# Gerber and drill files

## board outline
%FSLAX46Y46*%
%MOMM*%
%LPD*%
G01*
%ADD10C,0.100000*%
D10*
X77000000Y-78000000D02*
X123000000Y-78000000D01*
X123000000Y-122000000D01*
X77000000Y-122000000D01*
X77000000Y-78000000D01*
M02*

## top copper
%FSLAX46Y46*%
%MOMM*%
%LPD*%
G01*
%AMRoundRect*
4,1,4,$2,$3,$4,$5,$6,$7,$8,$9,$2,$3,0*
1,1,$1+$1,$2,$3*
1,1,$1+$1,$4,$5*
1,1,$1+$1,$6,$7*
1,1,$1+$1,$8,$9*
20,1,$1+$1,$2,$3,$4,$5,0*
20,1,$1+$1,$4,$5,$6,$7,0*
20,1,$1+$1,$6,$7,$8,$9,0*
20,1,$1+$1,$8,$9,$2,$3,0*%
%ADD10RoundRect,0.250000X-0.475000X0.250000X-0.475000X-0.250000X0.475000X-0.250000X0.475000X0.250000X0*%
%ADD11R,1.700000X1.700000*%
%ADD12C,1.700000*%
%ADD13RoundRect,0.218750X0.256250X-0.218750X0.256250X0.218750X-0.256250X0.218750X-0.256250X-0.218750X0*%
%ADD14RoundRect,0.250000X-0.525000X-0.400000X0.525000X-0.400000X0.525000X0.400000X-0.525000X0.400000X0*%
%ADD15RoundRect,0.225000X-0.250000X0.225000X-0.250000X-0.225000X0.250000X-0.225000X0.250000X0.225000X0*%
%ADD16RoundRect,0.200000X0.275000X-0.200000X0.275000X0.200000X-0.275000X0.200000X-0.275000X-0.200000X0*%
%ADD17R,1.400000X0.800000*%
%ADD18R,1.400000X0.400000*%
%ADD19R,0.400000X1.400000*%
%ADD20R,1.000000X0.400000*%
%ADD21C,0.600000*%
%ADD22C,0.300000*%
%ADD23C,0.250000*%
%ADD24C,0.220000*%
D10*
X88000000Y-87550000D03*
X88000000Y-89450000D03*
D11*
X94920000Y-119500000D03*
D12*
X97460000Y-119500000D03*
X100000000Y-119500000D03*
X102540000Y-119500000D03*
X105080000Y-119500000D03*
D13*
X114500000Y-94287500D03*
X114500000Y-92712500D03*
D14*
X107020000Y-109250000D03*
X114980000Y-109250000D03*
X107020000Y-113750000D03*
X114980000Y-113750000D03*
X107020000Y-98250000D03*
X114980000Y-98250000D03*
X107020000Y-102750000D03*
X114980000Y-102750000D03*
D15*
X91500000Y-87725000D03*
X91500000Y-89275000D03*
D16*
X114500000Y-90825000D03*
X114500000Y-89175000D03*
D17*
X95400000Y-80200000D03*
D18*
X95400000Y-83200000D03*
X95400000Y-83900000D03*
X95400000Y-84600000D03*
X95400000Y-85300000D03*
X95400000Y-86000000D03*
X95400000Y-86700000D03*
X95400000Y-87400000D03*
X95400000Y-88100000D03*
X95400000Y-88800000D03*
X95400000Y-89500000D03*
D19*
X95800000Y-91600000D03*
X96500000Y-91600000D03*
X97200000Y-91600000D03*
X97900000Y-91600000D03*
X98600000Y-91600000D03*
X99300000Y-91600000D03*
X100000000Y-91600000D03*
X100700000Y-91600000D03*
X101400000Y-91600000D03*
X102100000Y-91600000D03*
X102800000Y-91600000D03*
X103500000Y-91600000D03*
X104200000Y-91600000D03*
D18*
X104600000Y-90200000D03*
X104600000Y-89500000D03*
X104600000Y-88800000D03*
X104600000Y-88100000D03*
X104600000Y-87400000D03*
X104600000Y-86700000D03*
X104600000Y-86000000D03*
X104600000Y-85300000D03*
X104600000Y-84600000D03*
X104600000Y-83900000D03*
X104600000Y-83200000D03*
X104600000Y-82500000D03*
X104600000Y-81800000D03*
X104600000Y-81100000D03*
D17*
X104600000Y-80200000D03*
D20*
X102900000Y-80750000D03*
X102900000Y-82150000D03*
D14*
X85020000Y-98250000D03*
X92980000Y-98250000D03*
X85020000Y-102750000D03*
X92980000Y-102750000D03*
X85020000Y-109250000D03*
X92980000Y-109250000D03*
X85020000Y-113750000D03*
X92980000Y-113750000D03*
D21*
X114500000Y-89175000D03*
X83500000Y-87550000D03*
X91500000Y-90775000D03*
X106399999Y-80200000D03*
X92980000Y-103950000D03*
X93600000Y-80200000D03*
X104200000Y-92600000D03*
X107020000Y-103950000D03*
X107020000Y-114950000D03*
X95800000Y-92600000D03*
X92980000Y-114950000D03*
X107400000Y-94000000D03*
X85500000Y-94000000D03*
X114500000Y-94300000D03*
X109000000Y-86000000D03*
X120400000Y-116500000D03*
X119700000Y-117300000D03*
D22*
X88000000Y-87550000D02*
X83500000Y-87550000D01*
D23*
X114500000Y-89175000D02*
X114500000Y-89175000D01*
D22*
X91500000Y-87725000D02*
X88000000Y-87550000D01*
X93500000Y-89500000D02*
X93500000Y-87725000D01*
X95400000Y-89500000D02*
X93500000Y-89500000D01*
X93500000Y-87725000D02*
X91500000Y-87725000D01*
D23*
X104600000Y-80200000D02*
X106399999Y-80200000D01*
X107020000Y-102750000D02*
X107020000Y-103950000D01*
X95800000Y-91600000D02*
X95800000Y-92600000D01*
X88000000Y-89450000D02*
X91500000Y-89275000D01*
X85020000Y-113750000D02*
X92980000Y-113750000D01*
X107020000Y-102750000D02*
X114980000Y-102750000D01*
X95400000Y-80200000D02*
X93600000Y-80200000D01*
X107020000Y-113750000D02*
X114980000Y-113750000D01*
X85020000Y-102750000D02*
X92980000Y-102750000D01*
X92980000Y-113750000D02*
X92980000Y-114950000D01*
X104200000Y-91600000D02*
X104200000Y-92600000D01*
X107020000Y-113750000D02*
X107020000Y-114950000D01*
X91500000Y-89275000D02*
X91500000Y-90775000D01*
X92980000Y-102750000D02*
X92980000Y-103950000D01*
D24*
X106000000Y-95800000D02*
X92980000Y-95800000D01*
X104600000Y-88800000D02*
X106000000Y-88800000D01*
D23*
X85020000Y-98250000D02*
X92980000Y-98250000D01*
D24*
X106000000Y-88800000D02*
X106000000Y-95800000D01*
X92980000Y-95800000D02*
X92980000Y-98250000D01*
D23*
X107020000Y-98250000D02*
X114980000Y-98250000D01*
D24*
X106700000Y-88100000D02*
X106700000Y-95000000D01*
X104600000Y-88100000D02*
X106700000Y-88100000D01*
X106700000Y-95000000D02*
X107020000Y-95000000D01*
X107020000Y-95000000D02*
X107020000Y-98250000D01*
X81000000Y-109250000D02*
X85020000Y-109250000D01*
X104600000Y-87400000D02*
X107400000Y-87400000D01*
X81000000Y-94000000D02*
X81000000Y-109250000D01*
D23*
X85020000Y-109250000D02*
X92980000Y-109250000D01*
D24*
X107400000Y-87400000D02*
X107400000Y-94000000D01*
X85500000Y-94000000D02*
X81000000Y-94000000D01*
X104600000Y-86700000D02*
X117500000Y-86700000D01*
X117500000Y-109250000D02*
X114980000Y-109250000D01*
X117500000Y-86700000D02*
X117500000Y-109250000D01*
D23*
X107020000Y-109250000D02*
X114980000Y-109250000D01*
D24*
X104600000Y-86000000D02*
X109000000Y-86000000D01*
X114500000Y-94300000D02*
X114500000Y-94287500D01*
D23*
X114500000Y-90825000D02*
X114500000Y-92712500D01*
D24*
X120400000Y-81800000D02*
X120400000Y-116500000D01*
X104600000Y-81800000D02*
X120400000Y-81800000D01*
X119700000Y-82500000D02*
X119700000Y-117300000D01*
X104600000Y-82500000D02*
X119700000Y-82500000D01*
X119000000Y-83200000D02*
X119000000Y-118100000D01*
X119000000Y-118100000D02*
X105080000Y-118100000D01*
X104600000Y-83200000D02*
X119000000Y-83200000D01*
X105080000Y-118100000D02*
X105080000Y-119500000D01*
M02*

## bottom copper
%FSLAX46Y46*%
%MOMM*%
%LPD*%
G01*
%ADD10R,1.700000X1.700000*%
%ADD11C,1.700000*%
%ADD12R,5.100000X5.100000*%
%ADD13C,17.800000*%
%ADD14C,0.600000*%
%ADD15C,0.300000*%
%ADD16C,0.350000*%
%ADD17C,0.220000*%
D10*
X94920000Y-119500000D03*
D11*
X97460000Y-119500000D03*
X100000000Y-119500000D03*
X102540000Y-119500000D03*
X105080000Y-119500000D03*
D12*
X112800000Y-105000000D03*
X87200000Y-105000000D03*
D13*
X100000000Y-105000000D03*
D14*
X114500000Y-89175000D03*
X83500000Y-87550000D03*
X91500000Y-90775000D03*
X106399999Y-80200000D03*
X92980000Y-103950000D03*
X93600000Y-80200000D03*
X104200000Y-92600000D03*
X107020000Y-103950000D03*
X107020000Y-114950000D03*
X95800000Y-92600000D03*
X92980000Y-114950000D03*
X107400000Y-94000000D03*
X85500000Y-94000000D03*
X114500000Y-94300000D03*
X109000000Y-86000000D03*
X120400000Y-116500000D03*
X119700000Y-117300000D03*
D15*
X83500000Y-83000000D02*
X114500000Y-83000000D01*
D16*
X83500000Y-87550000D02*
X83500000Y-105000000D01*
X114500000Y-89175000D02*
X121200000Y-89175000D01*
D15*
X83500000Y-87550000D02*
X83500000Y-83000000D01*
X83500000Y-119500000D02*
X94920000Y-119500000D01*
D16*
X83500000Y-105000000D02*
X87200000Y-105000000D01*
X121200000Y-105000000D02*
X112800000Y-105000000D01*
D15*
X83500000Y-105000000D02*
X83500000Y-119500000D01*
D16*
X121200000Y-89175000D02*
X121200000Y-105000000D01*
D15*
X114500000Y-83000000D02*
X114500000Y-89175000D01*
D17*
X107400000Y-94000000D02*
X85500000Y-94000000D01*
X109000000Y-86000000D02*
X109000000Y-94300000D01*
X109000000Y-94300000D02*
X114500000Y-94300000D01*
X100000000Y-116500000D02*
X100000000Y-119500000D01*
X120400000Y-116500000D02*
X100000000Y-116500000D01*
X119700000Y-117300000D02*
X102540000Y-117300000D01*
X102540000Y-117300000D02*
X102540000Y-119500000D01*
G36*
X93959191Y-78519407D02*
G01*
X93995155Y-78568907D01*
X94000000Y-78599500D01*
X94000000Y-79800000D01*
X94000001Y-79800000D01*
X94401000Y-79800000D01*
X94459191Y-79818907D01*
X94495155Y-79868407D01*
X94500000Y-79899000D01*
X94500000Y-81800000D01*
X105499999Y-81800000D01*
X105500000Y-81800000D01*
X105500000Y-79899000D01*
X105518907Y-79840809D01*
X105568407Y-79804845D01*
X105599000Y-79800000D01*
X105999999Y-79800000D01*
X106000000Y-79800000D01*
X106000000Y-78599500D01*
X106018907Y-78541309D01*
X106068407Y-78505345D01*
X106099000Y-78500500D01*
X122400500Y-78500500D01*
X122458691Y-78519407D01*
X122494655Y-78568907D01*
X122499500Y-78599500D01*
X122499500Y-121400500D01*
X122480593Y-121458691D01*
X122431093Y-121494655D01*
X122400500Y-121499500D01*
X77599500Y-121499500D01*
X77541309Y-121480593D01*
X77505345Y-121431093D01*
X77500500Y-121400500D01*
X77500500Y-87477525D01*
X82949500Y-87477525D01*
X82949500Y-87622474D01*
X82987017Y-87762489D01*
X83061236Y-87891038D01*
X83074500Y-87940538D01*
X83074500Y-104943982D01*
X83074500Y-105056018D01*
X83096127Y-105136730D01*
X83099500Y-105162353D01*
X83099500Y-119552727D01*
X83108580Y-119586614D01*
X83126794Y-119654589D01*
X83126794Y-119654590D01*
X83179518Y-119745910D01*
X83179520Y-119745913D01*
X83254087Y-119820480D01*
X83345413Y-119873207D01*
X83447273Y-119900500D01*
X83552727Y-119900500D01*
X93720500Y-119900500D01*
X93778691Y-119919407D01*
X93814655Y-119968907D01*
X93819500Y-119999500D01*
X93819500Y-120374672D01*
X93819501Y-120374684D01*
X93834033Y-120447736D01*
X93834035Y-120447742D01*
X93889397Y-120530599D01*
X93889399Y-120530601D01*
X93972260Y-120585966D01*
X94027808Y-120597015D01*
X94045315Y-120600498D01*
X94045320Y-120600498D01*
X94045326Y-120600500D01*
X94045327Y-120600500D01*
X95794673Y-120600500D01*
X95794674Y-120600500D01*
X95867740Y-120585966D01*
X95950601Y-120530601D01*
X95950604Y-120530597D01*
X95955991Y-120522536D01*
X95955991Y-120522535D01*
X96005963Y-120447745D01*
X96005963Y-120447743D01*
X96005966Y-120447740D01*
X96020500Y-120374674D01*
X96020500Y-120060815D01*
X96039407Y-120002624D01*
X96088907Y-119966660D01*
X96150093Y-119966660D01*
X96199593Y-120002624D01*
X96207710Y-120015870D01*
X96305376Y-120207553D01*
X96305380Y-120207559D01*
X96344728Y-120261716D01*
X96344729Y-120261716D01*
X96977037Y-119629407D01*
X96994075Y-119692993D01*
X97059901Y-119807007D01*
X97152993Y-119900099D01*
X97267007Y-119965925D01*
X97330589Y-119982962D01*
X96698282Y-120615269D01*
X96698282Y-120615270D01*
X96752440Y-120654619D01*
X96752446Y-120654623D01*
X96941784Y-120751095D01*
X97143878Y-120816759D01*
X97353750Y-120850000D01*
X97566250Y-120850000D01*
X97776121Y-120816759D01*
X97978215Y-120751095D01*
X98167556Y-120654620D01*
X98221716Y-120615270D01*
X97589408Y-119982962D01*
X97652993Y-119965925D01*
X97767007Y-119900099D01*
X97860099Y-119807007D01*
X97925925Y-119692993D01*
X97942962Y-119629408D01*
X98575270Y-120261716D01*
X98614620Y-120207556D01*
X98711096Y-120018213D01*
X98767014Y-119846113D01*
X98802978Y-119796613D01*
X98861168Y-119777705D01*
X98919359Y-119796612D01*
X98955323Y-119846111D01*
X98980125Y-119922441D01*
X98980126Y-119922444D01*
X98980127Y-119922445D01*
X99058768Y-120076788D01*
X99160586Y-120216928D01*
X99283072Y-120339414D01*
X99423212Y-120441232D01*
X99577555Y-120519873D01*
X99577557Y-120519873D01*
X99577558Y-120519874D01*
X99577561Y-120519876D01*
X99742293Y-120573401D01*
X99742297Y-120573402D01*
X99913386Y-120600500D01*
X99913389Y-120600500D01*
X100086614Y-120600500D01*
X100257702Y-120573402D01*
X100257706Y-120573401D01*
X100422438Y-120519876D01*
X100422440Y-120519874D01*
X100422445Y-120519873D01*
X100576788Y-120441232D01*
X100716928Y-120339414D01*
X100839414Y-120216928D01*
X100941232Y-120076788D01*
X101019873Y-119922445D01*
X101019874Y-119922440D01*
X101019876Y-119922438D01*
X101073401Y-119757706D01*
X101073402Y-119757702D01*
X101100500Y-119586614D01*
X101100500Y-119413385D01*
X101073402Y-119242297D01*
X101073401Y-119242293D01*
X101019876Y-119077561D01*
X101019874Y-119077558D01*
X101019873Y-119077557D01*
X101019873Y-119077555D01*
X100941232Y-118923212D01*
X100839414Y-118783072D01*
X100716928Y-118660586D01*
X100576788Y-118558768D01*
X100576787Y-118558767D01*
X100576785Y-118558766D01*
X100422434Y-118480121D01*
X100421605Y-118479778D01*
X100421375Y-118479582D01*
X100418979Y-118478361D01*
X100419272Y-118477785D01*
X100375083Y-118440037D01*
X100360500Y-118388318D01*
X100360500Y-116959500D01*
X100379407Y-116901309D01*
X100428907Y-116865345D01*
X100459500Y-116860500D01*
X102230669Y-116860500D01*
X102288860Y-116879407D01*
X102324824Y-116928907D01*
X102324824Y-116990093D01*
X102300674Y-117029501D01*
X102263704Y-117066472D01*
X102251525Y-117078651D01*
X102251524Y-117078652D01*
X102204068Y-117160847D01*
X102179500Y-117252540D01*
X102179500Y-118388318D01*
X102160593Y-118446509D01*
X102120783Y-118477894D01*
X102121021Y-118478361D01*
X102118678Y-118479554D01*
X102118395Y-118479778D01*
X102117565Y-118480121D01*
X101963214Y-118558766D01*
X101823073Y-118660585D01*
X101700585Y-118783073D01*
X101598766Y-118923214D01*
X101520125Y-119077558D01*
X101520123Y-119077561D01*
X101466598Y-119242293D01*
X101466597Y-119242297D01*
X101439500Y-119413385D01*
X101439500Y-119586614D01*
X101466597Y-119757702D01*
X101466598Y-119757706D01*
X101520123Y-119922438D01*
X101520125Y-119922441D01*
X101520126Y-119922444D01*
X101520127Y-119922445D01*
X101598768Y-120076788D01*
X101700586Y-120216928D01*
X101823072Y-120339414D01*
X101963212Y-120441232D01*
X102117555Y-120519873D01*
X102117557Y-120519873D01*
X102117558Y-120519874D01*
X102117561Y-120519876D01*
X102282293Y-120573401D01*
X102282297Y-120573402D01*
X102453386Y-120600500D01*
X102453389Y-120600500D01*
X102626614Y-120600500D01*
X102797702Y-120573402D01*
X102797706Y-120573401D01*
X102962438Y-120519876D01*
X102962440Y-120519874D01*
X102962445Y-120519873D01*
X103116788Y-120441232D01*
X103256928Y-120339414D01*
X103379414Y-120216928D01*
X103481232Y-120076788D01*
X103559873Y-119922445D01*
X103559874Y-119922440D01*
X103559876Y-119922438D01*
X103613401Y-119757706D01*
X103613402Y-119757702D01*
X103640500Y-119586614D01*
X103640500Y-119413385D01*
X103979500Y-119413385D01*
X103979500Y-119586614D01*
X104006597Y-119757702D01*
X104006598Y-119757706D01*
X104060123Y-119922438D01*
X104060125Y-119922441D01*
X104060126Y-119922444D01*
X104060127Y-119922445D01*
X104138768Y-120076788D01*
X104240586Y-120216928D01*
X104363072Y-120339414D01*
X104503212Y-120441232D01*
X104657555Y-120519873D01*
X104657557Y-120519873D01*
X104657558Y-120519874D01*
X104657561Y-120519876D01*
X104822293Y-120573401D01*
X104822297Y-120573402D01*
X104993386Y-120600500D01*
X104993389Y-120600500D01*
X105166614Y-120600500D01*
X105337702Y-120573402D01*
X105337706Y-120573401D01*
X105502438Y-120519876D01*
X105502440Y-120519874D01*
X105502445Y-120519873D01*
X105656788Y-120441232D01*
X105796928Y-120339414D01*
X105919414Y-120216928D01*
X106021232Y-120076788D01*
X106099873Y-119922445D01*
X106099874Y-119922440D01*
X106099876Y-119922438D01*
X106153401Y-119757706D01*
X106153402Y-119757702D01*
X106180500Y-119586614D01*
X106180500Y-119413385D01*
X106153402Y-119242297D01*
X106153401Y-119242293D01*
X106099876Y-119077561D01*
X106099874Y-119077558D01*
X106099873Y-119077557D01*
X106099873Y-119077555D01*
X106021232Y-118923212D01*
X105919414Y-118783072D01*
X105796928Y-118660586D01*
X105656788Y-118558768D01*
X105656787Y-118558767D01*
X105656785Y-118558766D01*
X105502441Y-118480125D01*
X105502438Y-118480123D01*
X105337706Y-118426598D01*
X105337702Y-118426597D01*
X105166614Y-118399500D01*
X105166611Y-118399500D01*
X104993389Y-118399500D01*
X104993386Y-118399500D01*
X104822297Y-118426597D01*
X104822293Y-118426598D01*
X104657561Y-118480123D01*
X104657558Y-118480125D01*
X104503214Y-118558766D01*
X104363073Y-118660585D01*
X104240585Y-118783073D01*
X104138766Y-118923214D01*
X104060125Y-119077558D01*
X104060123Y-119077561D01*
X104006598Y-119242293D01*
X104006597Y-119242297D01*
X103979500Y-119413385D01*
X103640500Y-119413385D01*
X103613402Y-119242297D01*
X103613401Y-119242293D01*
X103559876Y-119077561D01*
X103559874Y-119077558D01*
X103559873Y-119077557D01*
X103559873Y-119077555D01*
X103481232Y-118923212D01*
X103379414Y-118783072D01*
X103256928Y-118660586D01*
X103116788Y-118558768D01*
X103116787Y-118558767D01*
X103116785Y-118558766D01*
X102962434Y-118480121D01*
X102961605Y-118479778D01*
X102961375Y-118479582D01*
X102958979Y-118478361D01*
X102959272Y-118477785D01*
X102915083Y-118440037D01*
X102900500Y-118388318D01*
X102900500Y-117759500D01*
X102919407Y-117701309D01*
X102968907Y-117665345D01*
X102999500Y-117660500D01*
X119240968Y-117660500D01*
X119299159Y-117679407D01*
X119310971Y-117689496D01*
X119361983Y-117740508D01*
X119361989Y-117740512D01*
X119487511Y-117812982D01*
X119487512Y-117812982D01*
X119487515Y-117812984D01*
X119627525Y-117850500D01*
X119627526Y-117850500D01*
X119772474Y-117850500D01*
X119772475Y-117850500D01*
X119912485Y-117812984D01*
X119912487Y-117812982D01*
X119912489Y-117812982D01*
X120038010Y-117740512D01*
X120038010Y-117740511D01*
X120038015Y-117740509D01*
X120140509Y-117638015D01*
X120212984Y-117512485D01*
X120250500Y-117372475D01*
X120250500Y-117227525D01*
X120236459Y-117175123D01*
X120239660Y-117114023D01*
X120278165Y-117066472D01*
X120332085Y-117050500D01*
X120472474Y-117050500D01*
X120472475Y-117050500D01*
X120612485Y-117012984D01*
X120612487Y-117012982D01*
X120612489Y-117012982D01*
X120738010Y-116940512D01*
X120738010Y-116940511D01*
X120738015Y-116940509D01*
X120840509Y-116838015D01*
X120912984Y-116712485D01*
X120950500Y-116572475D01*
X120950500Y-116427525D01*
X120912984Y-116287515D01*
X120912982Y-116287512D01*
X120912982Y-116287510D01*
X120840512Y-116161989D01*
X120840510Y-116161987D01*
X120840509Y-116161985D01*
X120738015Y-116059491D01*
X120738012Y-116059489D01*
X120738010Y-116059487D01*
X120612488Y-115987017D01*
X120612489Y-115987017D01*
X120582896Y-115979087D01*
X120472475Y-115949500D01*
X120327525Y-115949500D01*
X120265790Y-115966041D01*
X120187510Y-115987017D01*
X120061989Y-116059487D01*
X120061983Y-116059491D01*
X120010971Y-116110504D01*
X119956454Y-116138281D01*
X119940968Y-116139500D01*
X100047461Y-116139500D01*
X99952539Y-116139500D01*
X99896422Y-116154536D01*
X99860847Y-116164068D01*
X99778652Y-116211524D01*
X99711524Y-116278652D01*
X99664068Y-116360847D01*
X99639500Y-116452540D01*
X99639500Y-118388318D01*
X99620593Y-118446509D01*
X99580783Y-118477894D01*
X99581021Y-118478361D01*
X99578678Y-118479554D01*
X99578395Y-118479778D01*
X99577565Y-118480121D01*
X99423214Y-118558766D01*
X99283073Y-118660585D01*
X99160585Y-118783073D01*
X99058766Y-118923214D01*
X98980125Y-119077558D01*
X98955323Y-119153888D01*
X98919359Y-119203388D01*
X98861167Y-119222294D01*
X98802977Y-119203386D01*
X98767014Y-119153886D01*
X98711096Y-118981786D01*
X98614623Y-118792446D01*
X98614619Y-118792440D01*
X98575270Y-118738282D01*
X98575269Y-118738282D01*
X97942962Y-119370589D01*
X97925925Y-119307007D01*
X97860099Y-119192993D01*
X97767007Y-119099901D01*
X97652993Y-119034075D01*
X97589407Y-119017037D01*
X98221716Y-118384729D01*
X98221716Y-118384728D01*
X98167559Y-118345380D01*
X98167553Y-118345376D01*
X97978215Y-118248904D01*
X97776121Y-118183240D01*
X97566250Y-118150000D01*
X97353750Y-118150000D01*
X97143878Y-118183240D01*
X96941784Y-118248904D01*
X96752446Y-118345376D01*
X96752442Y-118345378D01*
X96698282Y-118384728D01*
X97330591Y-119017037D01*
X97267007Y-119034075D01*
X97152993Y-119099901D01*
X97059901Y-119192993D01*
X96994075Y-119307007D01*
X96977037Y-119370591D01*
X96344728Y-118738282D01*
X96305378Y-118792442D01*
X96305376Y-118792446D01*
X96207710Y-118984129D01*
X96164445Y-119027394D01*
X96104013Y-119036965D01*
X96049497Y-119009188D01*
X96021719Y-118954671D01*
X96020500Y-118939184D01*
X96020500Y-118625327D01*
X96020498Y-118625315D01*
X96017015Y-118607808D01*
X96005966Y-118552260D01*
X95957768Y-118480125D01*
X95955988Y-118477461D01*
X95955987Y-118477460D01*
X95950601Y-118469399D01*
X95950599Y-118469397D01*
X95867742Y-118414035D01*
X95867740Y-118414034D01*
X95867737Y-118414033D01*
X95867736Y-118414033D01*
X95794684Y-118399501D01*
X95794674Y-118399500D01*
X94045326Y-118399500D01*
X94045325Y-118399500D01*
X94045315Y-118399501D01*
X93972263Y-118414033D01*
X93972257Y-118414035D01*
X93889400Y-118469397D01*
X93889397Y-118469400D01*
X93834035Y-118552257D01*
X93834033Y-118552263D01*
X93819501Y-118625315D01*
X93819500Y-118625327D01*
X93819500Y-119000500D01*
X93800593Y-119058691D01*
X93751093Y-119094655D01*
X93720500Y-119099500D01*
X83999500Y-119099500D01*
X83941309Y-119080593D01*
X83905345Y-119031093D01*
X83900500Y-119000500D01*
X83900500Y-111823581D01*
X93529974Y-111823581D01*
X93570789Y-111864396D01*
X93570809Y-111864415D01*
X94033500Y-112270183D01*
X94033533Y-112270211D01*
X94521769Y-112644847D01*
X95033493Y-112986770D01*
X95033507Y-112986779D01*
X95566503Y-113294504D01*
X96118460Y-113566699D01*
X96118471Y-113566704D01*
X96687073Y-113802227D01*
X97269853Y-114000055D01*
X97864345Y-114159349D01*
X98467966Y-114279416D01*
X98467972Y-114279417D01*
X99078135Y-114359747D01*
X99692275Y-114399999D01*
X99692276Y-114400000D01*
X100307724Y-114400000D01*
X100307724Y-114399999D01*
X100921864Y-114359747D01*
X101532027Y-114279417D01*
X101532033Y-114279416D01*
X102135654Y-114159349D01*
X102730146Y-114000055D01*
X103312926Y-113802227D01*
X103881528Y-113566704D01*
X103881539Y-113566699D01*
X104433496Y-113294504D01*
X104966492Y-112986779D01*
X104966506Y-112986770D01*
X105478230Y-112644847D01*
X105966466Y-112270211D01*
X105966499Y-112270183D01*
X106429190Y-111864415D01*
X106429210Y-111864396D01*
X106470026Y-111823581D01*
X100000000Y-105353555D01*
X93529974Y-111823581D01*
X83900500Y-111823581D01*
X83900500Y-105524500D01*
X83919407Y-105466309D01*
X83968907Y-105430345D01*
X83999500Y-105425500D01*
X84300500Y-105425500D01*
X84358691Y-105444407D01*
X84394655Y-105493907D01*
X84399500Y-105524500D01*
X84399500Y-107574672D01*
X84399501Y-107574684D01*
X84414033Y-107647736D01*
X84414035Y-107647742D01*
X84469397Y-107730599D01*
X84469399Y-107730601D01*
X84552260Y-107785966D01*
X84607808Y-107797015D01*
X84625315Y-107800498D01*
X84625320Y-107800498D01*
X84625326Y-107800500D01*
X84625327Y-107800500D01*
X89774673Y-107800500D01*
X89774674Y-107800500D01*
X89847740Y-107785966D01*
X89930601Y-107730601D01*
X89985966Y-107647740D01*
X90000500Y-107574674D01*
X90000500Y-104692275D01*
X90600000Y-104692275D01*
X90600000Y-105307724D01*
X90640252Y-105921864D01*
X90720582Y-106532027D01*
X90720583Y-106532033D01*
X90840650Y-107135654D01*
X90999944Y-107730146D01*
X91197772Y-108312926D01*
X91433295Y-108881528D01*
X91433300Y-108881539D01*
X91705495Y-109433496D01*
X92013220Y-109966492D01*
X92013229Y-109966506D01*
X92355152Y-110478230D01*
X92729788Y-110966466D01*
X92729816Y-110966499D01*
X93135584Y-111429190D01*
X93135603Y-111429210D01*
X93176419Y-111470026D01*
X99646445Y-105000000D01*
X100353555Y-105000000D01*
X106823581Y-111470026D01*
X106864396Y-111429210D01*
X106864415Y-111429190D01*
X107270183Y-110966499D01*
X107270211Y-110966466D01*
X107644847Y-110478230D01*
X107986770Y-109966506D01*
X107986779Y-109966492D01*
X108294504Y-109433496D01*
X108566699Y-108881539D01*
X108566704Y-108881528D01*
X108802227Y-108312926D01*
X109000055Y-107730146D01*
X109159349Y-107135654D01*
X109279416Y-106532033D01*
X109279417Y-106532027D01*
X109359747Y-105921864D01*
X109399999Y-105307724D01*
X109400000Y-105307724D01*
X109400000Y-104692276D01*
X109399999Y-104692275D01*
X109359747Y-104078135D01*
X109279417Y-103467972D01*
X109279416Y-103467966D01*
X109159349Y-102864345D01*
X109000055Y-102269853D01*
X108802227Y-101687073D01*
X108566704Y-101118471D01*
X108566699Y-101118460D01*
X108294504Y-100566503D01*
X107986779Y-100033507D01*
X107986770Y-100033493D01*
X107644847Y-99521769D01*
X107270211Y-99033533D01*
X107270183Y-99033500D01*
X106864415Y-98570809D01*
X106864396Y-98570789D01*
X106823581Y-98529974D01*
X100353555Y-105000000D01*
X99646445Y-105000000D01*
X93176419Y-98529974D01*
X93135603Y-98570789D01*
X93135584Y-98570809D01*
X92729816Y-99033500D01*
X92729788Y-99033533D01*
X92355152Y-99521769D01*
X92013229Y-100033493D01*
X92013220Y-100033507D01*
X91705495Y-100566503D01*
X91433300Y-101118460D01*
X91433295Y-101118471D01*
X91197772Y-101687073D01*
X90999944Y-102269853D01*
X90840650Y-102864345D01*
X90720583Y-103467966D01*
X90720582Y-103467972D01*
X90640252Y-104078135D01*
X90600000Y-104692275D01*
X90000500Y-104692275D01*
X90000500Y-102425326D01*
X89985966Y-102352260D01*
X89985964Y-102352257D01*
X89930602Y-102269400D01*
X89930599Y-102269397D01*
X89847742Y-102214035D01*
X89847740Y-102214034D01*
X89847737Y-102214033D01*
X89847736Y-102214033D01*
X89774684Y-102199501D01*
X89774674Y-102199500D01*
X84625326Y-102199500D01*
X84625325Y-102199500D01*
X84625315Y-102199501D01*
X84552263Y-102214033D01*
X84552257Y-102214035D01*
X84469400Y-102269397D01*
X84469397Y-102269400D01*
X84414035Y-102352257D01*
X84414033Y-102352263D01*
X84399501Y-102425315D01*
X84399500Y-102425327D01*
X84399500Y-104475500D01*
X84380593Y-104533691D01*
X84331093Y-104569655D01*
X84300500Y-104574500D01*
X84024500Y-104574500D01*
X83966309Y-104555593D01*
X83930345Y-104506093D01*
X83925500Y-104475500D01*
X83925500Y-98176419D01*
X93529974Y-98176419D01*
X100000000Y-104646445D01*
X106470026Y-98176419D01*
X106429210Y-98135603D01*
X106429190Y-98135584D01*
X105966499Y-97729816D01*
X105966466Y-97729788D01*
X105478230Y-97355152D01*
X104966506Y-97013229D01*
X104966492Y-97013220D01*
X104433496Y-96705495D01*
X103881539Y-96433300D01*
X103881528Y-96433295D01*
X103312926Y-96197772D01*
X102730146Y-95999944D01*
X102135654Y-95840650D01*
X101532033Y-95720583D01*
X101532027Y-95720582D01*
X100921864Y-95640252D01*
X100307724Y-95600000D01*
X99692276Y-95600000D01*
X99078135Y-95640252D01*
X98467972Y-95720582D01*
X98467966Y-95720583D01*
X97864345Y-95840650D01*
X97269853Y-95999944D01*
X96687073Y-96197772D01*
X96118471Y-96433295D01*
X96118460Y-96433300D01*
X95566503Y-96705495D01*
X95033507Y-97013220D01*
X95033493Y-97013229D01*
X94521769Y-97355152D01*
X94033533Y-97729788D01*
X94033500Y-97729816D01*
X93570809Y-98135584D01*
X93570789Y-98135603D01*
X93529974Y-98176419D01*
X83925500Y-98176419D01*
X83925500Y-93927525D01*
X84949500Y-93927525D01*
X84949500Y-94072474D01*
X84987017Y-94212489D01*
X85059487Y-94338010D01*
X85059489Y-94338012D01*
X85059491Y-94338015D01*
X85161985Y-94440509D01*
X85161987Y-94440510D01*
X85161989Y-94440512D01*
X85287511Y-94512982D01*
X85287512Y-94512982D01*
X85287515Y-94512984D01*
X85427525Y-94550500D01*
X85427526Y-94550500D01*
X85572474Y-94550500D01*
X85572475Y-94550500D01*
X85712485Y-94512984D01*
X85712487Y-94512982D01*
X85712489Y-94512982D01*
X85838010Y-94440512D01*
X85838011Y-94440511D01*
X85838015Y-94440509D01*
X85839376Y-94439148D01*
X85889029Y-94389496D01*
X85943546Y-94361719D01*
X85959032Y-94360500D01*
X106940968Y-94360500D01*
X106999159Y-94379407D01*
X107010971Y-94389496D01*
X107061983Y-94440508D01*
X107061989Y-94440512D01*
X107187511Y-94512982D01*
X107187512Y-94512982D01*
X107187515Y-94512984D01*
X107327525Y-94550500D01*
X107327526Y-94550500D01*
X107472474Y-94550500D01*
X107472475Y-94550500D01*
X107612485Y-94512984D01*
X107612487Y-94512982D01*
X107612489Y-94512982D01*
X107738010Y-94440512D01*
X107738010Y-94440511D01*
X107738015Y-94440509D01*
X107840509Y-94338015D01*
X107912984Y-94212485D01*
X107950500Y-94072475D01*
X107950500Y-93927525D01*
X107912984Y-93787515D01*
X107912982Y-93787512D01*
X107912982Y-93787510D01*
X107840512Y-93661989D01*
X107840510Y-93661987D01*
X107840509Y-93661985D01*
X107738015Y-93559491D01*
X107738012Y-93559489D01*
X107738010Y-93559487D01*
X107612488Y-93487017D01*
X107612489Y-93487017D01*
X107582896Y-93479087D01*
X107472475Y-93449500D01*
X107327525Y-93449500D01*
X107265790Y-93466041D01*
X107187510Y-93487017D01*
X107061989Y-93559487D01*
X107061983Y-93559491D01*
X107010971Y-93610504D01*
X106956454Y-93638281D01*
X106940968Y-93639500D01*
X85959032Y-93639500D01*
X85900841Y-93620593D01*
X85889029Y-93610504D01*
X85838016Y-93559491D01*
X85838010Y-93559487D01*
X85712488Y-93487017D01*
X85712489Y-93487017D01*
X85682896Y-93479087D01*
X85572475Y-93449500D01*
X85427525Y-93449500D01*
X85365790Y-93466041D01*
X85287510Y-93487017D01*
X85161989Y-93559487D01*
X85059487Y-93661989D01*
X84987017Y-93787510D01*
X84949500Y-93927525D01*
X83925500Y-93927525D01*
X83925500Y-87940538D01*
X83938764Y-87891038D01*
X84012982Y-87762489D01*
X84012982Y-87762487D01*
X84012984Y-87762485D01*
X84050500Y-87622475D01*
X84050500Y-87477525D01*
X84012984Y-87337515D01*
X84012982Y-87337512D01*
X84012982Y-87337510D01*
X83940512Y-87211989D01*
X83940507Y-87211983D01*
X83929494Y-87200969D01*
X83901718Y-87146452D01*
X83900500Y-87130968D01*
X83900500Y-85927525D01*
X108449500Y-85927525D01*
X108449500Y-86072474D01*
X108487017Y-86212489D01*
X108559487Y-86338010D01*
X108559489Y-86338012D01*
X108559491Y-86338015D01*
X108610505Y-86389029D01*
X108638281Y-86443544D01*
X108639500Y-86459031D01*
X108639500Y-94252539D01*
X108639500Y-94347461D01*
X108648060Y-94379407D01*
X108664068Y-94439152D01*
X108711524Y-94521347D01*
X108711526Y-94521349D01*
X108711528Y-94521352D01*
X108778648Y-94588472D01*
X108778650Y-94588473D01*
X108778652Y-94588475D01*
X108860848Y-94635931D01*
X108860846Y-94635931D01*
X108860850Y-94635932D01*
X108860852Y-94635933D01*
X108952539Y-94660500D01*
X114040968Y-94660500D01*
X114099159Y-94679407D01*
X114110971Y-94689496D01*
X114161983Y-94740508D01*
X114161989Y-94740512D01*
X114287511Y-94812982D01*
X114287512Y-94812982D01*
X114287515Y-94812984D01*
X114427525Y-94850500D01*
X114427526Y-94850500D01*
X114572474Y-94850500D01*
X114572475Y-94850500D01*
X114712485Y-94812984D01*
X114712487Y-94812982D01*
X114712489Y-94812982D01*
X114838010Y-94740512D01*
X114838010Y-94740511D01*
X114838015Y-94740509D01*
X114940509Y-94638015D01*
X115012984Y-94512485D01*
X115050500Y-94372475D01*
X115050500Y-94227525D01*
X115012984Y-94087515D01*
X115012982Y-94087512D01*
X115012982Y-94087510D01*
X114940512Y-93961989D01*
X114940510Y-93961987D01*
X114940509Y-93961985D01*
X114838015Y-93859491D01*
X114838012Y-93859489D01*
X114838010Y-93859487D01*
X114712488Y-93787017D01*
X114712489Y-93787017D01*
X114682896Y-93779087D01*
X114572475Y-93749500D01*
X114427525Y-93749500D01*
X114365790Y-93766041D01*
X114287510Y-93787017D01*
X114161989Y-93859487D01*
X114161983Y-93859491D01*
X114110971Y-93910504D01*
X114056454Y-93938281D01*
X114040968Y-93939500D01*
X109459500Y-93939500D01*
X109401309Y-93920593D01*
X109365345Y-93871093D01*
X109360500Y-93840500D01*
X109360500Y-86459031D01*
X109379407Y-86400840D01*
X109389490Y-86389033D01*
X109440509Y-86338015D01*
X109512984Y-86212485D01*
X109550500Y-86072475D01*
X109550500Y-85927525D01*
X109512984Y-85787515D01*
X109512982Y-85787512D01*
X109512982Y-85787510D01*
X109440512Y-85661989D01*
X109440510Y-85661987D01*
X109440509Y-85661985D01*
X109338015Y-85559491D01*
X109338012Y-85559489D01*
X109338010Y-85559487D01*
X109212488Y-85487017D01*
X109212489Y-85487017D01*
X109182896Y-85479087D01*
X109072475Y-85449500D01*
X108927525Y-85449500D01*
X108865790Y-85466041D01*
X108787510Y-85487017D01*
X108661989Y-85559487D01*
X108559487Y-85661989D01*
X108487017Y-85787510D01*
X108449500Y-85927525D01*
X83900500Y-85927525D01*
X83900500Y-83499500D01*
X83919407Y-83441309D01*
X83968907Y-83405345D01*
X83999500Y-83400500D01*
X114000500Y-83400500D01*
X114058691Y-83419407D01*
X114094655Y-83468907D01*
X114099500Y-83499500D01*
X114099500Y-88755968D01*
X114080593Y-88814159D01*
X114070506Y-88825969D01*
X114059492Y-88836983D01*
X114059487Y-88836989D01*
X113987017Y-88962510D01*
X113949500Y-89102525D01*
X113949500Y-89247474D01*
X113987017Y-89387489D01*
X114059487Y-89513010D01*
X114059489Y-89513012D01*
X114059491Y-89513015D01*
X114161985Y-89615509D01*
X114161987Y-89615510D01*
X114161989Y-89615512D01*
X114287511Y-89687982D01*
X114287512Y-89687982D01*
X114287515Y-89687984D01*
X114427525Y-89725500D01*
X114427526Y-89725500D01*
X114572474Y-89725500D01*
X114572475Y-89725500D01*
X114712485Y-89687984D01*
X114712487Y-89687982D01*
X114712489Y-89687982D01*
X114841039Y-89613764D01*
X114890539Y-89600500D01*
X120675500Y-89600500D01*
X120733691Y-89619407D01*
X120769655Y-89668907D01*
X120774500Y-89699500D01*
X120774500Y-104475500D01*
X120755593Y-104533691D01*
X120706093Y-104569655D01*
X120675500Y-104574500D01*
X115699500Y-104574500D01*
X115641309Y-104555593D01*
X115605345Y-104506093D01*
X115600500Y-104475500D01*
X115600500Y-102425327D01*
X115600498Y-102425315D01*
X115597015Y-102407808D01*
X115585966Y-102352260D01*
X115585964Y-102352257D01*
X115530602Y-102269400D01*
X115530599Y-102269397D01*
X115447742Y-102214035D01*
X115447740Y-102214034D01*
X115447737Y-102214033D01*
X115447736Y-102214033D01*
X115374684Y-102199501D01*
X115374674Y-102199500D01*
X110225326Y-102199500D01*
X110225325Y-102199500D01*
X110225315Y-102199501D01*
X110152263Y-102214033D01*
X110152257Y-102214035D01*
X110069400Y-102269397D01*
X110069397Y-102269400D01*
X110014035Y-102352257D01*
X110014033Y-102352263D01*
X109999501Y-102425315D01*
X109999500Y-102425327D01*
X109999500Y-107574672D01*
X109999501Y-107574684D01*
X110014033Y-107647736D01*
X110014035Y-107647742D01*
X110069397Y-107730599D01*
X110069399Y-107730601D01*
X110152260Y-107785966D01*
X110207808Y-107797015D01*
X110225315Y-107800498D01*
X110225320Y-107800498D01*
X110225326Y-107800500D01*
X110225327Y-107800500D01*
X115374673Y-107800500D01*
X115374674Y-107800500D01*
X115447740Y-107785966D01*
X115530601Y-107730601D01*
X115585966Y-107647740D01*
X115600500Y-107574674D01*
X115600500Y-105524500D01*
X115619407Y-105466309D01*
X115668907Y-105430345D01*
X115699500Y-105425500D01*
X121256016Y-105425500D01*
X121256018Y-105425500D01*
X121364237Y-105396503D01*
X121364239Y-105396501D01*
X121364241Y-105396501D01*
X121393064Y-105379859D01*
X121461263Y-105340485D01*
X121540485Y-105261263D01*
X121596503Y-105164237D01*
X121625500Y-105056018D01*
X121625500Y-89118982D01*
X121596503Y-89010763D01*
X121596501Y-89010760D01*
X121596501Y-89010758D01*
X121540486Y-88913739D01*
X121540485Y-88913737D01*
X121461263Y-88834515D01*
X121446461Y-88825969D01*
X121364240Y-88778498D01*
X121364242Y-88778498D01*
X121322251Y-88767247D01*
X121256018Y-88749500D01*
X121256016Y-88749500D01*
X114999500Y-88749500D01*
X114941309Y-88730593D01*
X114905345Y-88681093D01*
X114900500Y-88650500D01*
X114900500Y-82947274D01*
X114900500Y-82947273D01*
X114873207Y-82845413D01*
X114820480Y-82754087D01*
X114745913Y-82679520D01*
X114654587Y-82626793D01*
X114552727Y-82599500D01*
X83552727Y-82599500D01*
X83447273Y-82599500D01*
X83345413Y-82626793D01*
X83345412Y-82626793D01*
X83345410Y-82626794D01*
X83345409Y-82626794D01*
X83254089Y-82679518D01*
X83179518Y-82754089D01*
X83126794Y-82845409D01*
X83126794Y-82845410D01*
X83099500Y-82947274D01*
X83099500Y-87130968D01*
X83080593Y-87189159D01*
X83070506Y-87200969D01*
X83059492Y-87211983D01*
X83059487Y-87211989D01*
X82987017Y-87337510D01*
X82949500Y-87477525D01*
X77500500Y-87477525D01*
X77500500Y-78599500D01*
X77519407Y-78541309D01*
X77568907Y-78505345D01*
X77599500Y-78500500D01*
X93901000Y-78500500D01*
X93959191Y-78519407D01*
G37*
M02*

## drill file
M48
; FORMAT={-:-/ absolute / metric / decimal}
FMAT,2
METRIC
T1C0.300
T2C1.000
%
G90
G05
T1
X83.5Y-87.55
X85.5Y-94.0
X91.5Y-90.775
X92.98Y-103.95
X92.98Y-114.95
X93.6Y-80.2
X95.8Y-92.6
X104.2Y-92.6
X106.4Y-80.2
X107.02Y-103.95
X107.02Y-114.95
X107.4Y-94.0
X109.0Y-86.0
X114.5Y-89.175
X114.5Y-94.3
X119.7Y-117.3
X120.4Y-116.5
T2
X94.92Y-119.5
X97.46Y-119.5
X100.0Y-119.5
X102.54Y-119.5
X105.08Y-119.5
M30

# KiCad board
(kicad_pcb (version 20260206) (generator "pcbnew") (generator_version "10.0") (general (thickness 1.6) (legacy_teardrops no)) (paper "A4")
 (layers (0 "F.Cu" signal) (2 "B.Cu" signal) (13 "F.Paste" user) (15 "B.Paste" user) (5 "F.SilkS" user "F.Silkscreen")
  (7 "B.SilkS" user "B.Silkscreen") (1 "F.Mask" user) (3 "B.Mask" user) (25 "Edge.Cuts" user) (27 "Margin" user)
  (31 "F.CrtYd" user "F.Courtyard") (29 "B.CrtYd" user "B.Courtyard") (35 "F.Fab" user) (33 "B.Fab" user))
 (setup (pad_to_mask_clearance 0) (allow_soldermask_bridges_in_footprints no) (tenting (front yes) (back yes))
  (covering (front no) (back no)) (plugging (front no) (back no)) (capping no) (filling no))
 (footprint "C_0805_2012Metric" (layer "F.Cu") (at 88 88.5 -90)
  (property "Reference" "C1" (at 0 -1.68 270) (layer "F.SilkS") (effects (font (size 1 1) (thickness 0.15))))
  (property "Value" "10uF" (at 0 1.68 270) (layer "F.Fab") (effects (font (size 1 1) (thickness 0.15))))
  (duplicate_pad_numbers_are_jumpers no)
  (pad "1" smd roundrect (at -0.95 0 270) (size 1 1.45) (layers "F.Cu" "F.Mask" "F.Paste") (roundrect_rratio 0.25) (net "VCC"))
  (pad "2" smd roundrect (at 0.95 0 270) (size 1 1.45) (layers "F.Cu" "F.Mask" "F.Paste") (roundrect_rratio 0.25) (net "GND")))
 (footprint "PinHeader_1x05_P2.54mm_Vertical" (layer "F.Cu") (at 94.92 119.5 90)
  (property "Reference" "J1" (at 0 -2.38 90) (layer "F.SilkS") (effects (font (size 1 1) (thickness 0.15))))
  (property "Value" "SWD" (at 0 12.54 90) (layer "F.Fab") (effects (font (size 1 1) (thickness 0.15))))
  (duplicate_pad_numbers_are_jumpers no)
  (pad "1" thru_hole rect (at 0 0 90) (size 1.7 1.7) (drill 1) (layers "*.Cu" "*.Mask") (remove_unused_layers no) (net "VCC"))
  (pad "2" thru_hole circle (at 0 2.54 90) (size 1.7 1.7) (drill 1) (layers "*.Cu" "*.Mask") (remove_unused_layers no) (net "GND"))
  (pad "3" thru_hole circle (at 0 5.08 90) (size 1.7 1.7) (drill 1) (layers "*.Cu" "*.Mask") (remove_unused_layers no) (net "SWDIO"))
  (pad "4" thru_hole circle (at 0 7.62 90) (size 1.7 1.7) (drill 1) (layers "*.Cu" "*.Mask") (remove_unused_layers no) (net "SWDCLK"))
  (pad "5" thru_hole circle (at 0 10.16 90) (size 1.7 1.7) (drill 1) (layers "*.Cu" "*.Mask") (remove_unused_layers no) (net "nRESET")))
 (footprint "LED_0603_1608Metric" (layer "F.Cu") (at 114.5 93.5 90)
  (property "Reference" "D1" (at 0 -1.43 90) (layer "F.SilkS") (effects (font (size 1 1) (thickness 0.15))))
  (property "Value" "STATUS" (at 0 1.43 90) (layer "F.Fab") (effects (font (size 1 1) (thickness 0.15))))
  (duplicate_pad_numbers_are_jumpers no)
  (pad "1" smd roundrect (at -0.7875 0 90) (size 0.875 0.95) (layers "F.Cu" "F.Mask" "F.Paste") (roundrect_rratio 0.25) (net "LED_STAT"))
  (pad "2" smd roundrect (at 0.7875 0 90) (size 0.875 0.95) (layers "F.Cu" "F.Mask" "F.Paste") (roundrect_rratio 0.25) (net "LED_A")))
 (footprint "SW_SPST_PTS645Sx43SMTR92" (layer "F.Cu") (at 111 111.5)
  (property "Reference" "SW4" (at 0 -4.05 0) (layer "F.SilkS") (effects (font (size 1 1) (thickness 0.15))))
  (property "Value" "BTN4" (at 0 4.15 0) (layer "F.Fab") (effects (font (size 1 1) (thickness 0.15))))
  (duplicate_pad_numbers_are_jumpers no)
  (pad "1" smd roundrect (at -3.98 -2.25) (size 1.55 1.3) (layers "F.Cu" "F.Mask" "F.Paste") (roundrect_rratio 0.1923076923) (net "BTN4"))
  (pad "1" smd roundrect (at 3.98 -2.25) (size 1.55 1.3) (layers "F.Cu" "F.Mask" "F.Paste") (roundrect_rratio 0.1923076923) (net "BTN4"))
  (pad "2" smd roundrect (at -3.98 2.25) (size 1.55 1.3) (layers "F.Cu" "F.Mask" "F.Paste") (roundrect_rratio 0.1923076923) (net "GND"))
  (pad "2" smd roundrect (at 3.98 2.25) (size 1.55 1.3) (layers "F.Cu" "F.Mask" "F.Paste") (roundrect_rratio 0.1923076923) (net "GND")))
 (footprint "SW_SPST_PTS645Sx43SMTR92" (layer "F.Cu") (at 111 100.5)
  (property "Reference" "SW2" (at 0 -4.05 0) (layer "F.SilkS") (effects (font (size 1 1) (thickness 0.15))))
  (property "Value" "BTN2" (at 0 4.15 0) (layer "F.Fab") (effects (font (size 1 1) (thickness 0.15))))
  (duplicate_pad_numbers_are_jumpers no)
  (pad "1" smd roundrect (at -3.98 -2.25) (size 1.55 1.3) (layers "F.Cu" "F.Mask" "F.Paste") (roundrect_rratio 0.1923076923) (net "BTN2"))
  (pad "1" smd roundrect (at 3.98 -2.25) (size 1.55 1.3) (layers "F.Cu" "F.Mask" "F.Paste") (roundrect_rratio 0.1923076923) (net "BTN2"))
  (pad "2" smd roundrect (at -3.98 2.25) (size 1.55 1.3) (layers "F.Cu" "F.Mask" "F.Paste") (roundrect_rratio 0.1923076923) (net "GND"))
  (pad "2" smd roundrect (at 3.98 2.25) (size 1.55 1.3) (layers "F.Cu" "F.Mask" "F.Paste") (roundrect_rratio 0.1923076923) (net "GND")))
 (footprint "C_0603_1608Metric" (layer "F.Cu") (at 91.5 88.5 -90)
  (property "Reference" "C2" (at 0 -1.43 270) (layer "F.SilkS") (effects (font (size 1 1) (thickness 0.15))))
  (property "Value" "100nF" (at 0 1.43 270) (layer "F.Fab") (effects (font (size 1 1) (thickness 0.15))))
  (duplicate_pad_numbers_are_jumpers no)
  (pad "1" smd roundrect (at -0.775 0 270) (size 0.9 0.95) (layers "F.Cu" "F.Mask" "F.Paste") (roundrect_rratio 0.25) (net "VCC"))
  (pad "2" smd roundrect (at 0.775 0 270) (size 0.9 0.95) (layers "F.Cu" "F.Mask" "F.Paste") (roundrect_rratio 0.25) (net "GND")))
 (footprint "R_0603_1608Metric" (layer "F.Cu") (at 114.5 90 90)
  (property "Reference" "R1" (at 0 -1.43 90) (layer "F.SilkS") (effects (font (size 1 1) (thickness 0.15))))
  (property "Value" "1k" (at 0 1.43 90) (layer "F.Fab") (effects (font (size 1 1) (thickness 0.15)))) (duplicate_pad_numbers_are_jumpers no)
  (pad "1" smd roundrect (at -0.825 0 90) (size 0.8 0.95) (layers "F.Cu" "F.Mask" "F.Paste") (roundrect_rratio 0.25) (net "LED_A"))
  (pad "2" smd roundrect (at 0.825 0 90) (size 0.8 0.95) (layers "F.Cu" "F.Mask" "F.Paste") (roundrect_rratio 0.25) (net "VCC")))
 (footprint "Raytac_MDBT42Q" (layer "F.Cu") (at 100 84)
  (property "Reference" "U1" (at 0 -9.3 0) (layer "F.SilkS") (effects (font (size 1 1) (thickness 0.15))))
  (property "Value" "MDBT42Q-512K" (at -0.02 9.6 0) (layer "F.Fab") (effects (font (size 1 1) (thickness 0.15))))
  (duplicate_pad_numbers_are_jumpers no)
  (pad "1" smd rect (at -4.6 -3.8) (size 1.4 0.8) (layers "F.Cu" "F.Mask" "F.Paste") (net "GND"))
  (pad "2" smd rect (at -4.6 -0.8) (size 1.4 0.4) (layers "F.Cu" "F.Mask" "F.Paste"))
  (pad "3" smd rect (at -4.6 -0.1) (size 1.4 0.4) (layers "F.Cu" "F.Mask" "F.Paste"))
  (pad "4" smd rect (at -4.6 0.6) (size 1.4 0.4) (layers "F.Cu" "F.Mask" "F.Paste"))
  (pad "5" smd rect (at -4.6 1.3) (size 1.4 0.4) (layers "F.Cu" "F.Mask" "F.Paste"))
  (pad "6" smd rect (at -4.6 2) (size 1.4 0.4) (layers "F.Cu" "F.Mask" "F.Paste"))
  (pad "7" smd rect (at -4.6 2.7) (size 1.4 0.4) (layers "F.Cu" "F.Mask" "F.Paste"))
  (pad "8" smd rect (at -4.6 3.4) (size 1.4 0.4) (layers "F.Cu" "F.Mask" "F.Paste"))
  (pad "9" smd rect (at -4.6 4.1) (size 1.4 0.4) (layers "F.Cu" "F.Mask" "F.Paste"))
  (pad "10" smd rect (at -4.6 4.8) (size 1.4 0.4) (layers "F.Cu" "F.Mask" "F.Paste"))
  (pad "11" smd rect (at -4.6 5.5) (size 1.4 0.4) (layers "F.Cu" "F.Mask" "F.Paste") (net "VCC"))
  (pad "12" smd rect (at -4.2 7.6 90) (size 1.4 0.4) (layers "F.Cu" "F.Mask" "F.Paste") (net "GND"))
  (pad "13" smd rect (at -3.5 7.6 90) (size 1.4 0.4) (layers "F.Cu" "F.Mask" "F.Paste"))
  (pad "14" smd rect (at -2.8 7.6 90) (size 1.4 0.4) (layers "F.Cu" "F.Mask" "F.Paste"))
  (pad "15" smd rect (at -2.1 7.6 90) (size 1.4 0.4) (layers "F.Cu" "F.Mask" "F.Paste"))
  (pad "16" smd rect (at -1.4 7.6 90) (size 1.4 0.4) (layers "F.Cu" "F.Mask" "F.Paste"))
  (pad "17" smd rect (at -0.7 7.6 90) (size 1.4 0.4) (layers "F.Cu" "F.Mask" "F.Paste"))
  (pad "18" smd rect (at 0 7.6 90) (size 1.4 0.4) (layers "F.Cu" "F.Mask" "F.Paste"))
  (pad "19" smd rect (at 0.7 7.6 90) (size 1.4 0.4) (layers "F.Cu" "F.Mask" "F.Paste"))
  (pad "20" smd rect (at 1.4 7.6 90) (size 1.4 0.4) (layers "F.Cu" "F.Mask" "F.Paste"))
  (pad "21" smd rect (at 2.1 7.6 90) (size 1.4 0.4) (layers "F.Cu" "F.Mask" "F.Paste"))
  (pad "22" smd rect (at 2.8 7.6 90) (size 1.4 0.4) (layers "F.Cu" "F.Mask" "F.Paste"))
  (pad "23" smd rect (at 3.5 7.6 90) (size 1.4 0.4) (layers "F.Cu" "F.Mask" "F.Paste"))
  (pad "24" smd rect (at 4.2 7.6 90) (size 1.4 0.4) (layers "F.Cu" "F.Mask" "F.Paste") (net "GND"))
  (pad "25" smd rect (at 4.6 6.2) (size 1.4 0.4) (layers "F.Cu" "F.Mask" "F.Paste"))
  (pad "26" smd rect (at 4.6 5.5) (size 1.4 0.4) (layers "F.Cu" "F.Mask" "F.Paste"))
  (pad "27" smd rect (at 4.6 4.8) (size 1.4 0.4) (layers "F.Cu" "F.Mask" "F.Paste") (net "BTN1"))
  (pad "28" smd rect (at 4.6 4.1) (size 1.4 0.4) (layers "F.Cu" "F.Mask" "F.Paste") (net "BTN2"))
  (pad "29" smd rect (at 4.6 3.4) (size 1.4 0.4) (layers "F.Cu" "F.Mask" "F.Paste") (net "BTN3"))
  (pad "30" smd rect (at 4.6 2.7) (size 1.4 0.4) (layers "F.Cu" "F.Mask" "F.Paste") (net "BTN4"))
  (pad "31" smd rect (at 4.6 2) (size 1.4 0.4) (layers "F.Cu" "F.Mask" "F.Paste") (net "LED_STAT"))
  (pad "32" smd rect (at 4.6 1.3) (size 1.4 0.4) (layers "F.Cu" "F.Mask" "F.Paste"))
  (pad "33" smd rect (at 4.6 0.6) (size 1.4 0.4) (layers "F.Cu" "F.Mask" "F.Paste"))
  (pad "34" smd rect (at 4.6 -0.1) (size 1.4 0.4) (layers "F.Cu" "F.Mask" "F.Paste"))
  (pad "35" smd rect (at 4.6 -0.8) (size 1.4 0.4) (layers "F.Cu" "F.Mask" "F.Paste") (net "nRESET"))
  (pad "36" smd rect (at 4.6 -1.5) (size 1.4 0.4) (layers "F.Cu" "F.Mask" "F.Paste") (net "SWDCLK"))
  (pad "37" smd rect (at 4.6 -2.2) (size 1.4 0.4) (layers "F.Cu" "F.Mask" "F.Paste") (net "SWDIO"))
  (pad "38" smd rect (at 4.6 -2.9) (size 1.4 0.4) (layers "F.Cu" "F.Mask" "F.Paste"))
  (pad "39" smd rect (at 4.6 -3.8) (size 1.4 0.8) (layers "F.Cu" "F.Mask" "F.Paste") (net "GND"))
  (pad "40" smd rect (at 2.9 -3.25) (size 1 0.4) (layers "F.Cu" "F.Mask" "F.Paste"))
  (pad "41" smd rect (at 2.9 -1.85) (size 1 0.4) (layers "F.Cu" "F.Mask" "F.Paste"))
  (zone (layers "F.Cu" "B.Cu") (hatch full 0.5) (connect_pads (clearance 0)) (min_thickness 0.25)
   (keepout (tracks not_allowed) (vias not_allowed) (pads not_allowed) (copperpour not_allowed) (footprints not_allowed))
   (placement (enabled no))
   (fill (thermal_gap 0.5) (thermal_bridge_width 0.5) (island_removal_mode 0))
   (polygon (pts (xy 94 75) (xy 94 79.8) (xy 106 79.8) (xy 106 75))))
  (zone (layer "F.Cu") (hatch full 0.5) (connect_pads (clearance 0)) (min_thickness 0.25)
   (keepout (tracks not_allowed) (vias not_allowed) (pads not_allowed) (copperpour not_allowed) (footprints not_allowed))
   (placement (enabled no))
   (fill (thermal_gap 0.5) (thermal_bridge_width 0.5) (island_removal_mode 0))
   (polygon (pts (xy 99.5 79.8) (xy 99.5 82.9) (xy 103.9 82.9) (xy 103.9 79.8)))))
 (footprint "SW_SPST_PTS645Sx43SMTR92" (layer "F.Cu") (at 89 100.5)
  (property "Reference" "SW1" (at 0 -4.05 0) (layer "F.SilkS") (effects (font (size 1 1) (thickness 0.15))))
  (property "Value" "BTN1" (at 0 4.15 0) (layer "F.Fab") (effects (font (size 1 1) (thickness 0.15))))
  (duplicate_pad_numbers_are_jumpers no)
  (pad "1" smd roundrect (at -3.98 -2.25) (size 1.55 1.3) (layers "F.Cu" "F.Mask" "F.Paste") (roundrect_rratio 0.1923076923) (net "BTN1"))
  (pad "1" smd roundrect (at 3.98 -2.25) (size 1.55 1.3) (layers "F.Cu" "F.Mask" "F.Paste") (roundrect_rratio 0.1923076923) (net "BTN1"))
  (pad "2" smd roundrect (at -3.98 2.25) (size 1.55 1.3) (layers "F.Cu" "F.Mask" "F.Paste") (roundrect_rratio 0.1923076923) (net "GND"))
  (pad "2" smd roundrect (at 3.98 2.25) (size 1.55 1.3) (layers "F.Cu" "F.Mask" "F.Paste") (roundrect_rratio 0.1923076923) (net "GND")))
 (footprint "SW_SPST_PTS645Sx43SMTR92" (layer "F.Cu") (at 89 111.5)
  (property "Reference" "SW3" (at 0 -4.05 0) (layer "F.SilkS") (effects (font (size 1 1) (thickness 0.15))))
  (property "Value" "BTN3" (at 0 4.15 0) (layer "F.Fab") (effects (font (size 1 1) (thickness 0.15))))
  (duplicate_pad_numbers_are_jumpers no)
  (pad "1" smd roundrect (at -3.98 -2.25) (size 1.55 1.3) (layers "F.Cu" "F.Mask" "F.Paste") (roundrect_rratio 0.1923076923) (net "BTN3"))
  (pad "1" smd roundrect (at 3.98 -2.25) (size 1.55 1.3) (layers "F.Cu" "F.Mask" "F.Paste") (roundrect_rratio 0.1923076923) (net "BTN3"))
  (pad "2" smd roundrect (at -3.98 2.25) (size 1.55 1.3) (layers "F.Cu" "F.Mask" "F.Paste") (roundrect_rratio 0.1923076923) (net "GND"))
  (pad "2" smd roundrect (at 3.98 2.25) (size 1.55 1.3) (layers "F.Cu" "F.Mask" "F.Paste") (roundrect_rratio 0.1923076923) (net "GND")))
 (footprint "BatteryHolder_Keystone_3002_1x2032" (layer "B.Cu") (at 100 105 180)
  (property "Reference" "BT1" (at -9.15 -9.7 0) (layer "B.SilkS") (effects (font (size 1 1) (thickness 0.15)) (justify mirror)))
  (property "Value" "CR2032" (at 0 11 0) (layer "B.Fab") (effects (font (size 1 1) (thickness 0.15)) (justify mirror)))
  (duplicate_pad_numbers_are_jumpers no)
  (pad "1" smd rect (at -12.8 0 180) (size 5.1 5.1) (layers "B.Cu" "B.Mask" "B.Paste") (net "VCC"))
  (pad "1" smd rect (at 12.8 0 180) (size 5.1 5.1) (layers "B.Cu" "B.Mask" "B.Paste") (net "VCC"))
  (pad "2" smd circle (at 0 0 180) (size 17.8 17.8) (layers "B.Cu" "B.Mask") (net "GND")))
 (gr_rect (start 77 78) (end 123 122) (stroke (width 0.1) (type default)) (fill no) (layer "Edge.Cuts"))
 (segment (start 88 87.55) (end 83.5 87.55) (width 0.3) (layer "F.Cu") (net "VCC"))
 (segment (start 114.5 89.175) (end 114.5 89.175) (width 0.25) (layer "F.Cu") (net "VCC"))
 (segment (start 91.5 87.725) (end 88 87.55) (width 0.3) (layer "F.Cu") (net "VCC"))
 (segment (start 93.5 89.5) (end 93.5 87.725) (width 0.3) (layer "F.Cu") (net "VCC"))
 (segment (start 95.4 89.5) (end 93.5 89.5) (width 0.3) (layer "F.Cu") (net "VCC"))
 (segment (start 93.5 87.725) (end 91.5 87.725) (width 0.3) (layer "F.Cu") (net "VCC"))
 (via (at 114.5 89.175) (size 0.6) (drill 0.3) (layers "F.Cu" "B.Cu") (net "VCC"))
 (via (at 83.5 87.55) (size 0.6) (drill 0.3) (layers "F.Cu" "B.Cu") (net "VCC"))
 (segment (start 83.5 83) (end 114.5 83) (width 0.3) (layer "B.Cu") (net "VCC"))
 (segment (start 83.5 87.55) (end 83.5 105) (width 0.35) (layer "B.Cu") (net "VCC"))
 (segment (start 114.5 89.175) (end 121.2 89.175) (width 0.35) (layer "B.Cu") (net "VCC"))
 (segment (start 83.5 87.55) (end 83.5 83) (width 0.3) (layer "B.Cu") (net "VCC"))
 (segment (start 83.5 119.5) (end 94.92 119.5) (width 0.3) (layer "B.Cu") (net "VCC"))
 (segment (start 83.5 105) (end 87.2 105) (width 0.35) (layer "B.Cu") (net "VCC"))
 (segment (start 121.2 105) (end 112.8 105) (width 0.35) (layer "B.Cu") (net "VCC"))
 (segment (start 83.5 105) (end 83.5 119.5) (width 0.3) (layer "B.Cu") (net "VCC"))
 (segment (start 121.2 89.175) (end 121.2 105) (width 0.35) (layer "B.Cu") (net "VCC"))
 (segment (start 114.5 83) (end 114.5 89.175) (width 0.3) (layer "B.Cu") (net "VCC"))
 (segment (start 104.6 80.2) (end 106.399999 80.2) (width 0.25) (layer "F.Cu") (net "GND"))
 (segment (start 107.02 102.75) (end 107.02 103.95) (width 0.25) (layer "F.Cu") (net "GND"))
 (segment (start 95.8 91.6) (end 95.8 92.6) (width 0.25) (layer "F.Cu") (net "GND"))
 (segment (start 88 89.45) (end 91.5 89.275) (width 0.25) (layer "F.Cu") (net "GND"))
 (segment (start 85.02 113.75) (end 92.98 113.75) (width 0.25) (layer "F.Cu") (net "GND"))
 (segment (start 107.02 102.75) (end 114.98 102.75) (width 0.25) (layer "F.Cu") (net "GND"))
 (segment (start 95.4 80.2) (end 93.6 80.2) (width 0.25) (layer "F.Cu") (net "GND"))
 (segment (start 107.02 113.75) (end 114.98 113.75) (width 0.25) (layer "F.Cu") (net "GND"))
 (segment (start 85.02 102.75) (end 92.98 102.75) (width 0.25) (layer "F.Cu") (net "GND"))
 (segment (start 92.98 113.75) (end 92.98 114.95) (width 0.25) (layer "F.Cu") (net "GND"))
 (segment (start 104.2 91.6) (end 104.2 92.6) (width 0.25) (layer "F.Cu") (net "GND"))
 (segment (start 107.02 113.75) (end 107.02 114.95) (width 0.25) (layer "F.Cu") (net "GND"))
 (segment (start 91.5 89.275) (end 91.5 90.775) (width 0.25) (layer "F.Cu") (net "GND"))
 (segment (start 92.98 102.75) (end 92.98 103.95) (width 0.25) (layer "F.Cu") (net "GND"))
 (via (at 91.5 90.775) (size 0.6) (drill 0.3) (layers "F.Cu" "B.Cu") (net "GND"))
 (via (at 106.399999 80.2) (size 0.6) (drill 0.3) (layers "F.Cu" "B.Cu") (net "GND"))
 (via (at 92.98 103.95) (size 0.6) (drill 0.3) (layers "F.Cu" "B.Cu") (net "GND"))
 (via (at 93.6 80.2) (size 0.6) (drill 0.3) (layers "F.Cu" "B.Cu") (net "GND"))
 (via (at 104.2 92.6) (size 0.6) (drill 0.3) (layers "F.Cu" "B.Cu") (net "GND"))
 (via (at 107.02 103.95) (size 0.6) (drill 0.3) (layers "F.Cu" "B.Cu") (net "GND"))
 (via (at 107.02 114.95) (size 0.6) (drill 0.3) (layers "F.Cu" "B.Cu") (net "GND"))
 (via (at 95.8 92.6) (size 0.6) (drill 0.3) (layers "F.Cu" "B.Cu") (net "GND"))
 (via (at 92.98 114.95) (size 0.6) (drill 0.3) (layers "F.Cu" "B.Cu") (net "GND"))
 (segment (start 106 95.8) (end 92.98 95.8) (width 0.22) (layer "F.Cu") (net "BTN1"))
 (segment (start 104.6 88.8) (end 106 88.8) (width 0.22) (layer "F.Cu") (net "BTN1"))
 (segment (start 85.02 98.25) (end 92.98 98.25) (width 0.25) (layer "F.Cu") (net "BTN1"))
 (segment (start 106 88.8) (end 106 95.8) (width 0.22) (layer "F.Cu") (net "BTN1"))
 (segment (start 92.98 95.8) (end 92.98 98.25) (width 0.22) (layer "F.Cu") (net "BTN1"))
 (segment (start 107.02 98.25) (end 114.98 98.25) (width 0.25) (layer "F.Cu") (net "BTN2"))
 (segment (start 106.7 88.1) (end 106.7 95) (width 0.22) (layer "F.Cu") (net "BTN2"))
 (segment (start 104.6 88.1) (end 106.7 88.1) (width 0.22) (layer "F.Cu") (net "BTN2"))
 (segment (start 106.7 95) (end 107.02 95) (width 0.22) (layer "F.Cu") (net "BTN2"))
 (segment (start 107.02 95) (end 107.02 98.25) (width 0.22) (layer "F.Cu") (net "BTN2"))
 (segment (start 81 109.25) (end 85.02 109.25) (width 0.22) (layer "F.Cu") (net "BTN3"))
 (segment (start 104.6 87.4) (end 107.4 87.4) (width 0.22) (layer "F.Cu") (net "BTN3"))
 (segment (start 81 94) (end 81 109.25) (width 0.22) (layer "F.Cu") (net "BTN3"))
 (segment (start 85.02 109.25) (end 92.98 109.25) (width 0.25) (layer "F.Cu") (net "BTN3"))
 (segment (start 107.4 87.4) (end 107.4 94) (width 0.22) (layer "F.Cu") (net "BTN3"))
 (segment (start 85.5 94) (end 81 94) (width 0.22) (layer "F.Cu") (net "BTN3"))
 (via (at 107.4 94) (size 0.6) (drill 0.3) (layers "F.Cu" "B.Cu") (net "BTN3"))
 (via (at 85.5 94) (size 0.6) (drill 0.3) (layers "F.Cu" "B.Cu") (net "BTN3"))
 (segment (start 107.4 94) (end 85.5 94) (width 0.22) (layer "B.Cu") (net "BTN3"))
 (segment (start 104.6 86.7) (end 117.5 86.7) (width 0.22) (layer "F.Cu") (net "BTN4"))
 (segment (start 117.5 109.25) (end 114.98 109.25) (width 0.22) (layer "F.Cu") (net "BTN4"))
 (segment (start 117.5 86.7) (end 117.5 109.25) (width 0.22) (layer "F.Cu") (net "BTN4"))
 (segment (start 107.02 109.25) (end 114.98 109.25) (width 0.25) (layer "F.Cu") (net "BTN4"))
 (segment (start 104.6 86) (end 109 86) (width 0.22) (layer "F.Cu") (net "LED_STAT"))
 (segment (start 114.5 94.3) (end 114.5 94.2875) (width 0.22) (layer "F.Cu") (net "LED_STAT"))
 (via (at 114.5 94.3) (size 0.6) (drill 0.3) (layers "F.Cu" "B.Cu") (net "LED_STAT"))
 (via (at 109 86) (size 0.6) (drill 0.3) (layers "F.Cu" "B.Cu") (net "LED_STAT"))
 (segment (start 109 86) (end 109 94.3) (width 0.22) (layer "B.Cu") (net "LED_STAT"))
 (segment (start 109 94.3) (end 114.5 94.3) (width 0.22) (layer "B.Cu") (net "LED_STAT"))
 (segment (start 114.5 90.825) (end 114.5 92.7125) (width 0.25) (layer "F.Cu") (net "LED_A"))
 (segment (start 120.4 81.8) (end 120.4 116.5) (width 0.22) (layer "F.Cu") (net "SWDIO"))
 (segment (start 104.6 81.8) (end 120.4 81.8) (width 0.22) (layer "F.Cu") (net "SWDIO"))
 (via (at 120.4 116.5) (size 0.6) (drill 0.3) (layers "F.Cu" "B.Cu") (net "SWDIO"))
 (segment (start 100 116.5) (end 100 119.5) (width 0.22) (layer "B.Cu") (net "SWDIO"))
 (segment (start 120.4 116.5) (end 100 116.5) (width 0.22) (layer "B.Cu") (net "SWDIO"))
 (segment (start 119.7 82.5) (end 119.7 117.3) (width 0.22) (layer "F.Cu") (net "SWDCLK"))
 (segment (start 104.6 82.5) (end 119.7 82.5) (width 0.22) (layer "F.Cu") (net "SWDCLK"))
 (via (at 119.7 117.3) (size 0.6) (drill 0.3) (layers "F.Cu" "B.Cu") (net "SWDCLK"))
 (segment (start 119.7 117.3) (end 102.54 117.3) (width 0.22) (layer "B.Cu") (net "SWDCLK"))
 (segment (start 102.54 117.3) (end 102.54 119.5) (width 0.22) (layer "B.Cu") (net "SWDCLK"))
 (segment (start 119 83.2) (end 119 118.1) (width 0.22) (layer "F.Cu") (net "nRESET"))
 (segment (start 119 118.1) (end 105.08 118.1) (width 0.22) (layer "F.Cu") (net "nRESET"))
 (segment (start 104.6 83.2) (end 119 83.2) (width 0.22) (layer "F.Cu") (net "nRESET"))
 (segment (start 105.08 118.1) (end 105.08 119.5) (width 0.22) (layer "F.Cu") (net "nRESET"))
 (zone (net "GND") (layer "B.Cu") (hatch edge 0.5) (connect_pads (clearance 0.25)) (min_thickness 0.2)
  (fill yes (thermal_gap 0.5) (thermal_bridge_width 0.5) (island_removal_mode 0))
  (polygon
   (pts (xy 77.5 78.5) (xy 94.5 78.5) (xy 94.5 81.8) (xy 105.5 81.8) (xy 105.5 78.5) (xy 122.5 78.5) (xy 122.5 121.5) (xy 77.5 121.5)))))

